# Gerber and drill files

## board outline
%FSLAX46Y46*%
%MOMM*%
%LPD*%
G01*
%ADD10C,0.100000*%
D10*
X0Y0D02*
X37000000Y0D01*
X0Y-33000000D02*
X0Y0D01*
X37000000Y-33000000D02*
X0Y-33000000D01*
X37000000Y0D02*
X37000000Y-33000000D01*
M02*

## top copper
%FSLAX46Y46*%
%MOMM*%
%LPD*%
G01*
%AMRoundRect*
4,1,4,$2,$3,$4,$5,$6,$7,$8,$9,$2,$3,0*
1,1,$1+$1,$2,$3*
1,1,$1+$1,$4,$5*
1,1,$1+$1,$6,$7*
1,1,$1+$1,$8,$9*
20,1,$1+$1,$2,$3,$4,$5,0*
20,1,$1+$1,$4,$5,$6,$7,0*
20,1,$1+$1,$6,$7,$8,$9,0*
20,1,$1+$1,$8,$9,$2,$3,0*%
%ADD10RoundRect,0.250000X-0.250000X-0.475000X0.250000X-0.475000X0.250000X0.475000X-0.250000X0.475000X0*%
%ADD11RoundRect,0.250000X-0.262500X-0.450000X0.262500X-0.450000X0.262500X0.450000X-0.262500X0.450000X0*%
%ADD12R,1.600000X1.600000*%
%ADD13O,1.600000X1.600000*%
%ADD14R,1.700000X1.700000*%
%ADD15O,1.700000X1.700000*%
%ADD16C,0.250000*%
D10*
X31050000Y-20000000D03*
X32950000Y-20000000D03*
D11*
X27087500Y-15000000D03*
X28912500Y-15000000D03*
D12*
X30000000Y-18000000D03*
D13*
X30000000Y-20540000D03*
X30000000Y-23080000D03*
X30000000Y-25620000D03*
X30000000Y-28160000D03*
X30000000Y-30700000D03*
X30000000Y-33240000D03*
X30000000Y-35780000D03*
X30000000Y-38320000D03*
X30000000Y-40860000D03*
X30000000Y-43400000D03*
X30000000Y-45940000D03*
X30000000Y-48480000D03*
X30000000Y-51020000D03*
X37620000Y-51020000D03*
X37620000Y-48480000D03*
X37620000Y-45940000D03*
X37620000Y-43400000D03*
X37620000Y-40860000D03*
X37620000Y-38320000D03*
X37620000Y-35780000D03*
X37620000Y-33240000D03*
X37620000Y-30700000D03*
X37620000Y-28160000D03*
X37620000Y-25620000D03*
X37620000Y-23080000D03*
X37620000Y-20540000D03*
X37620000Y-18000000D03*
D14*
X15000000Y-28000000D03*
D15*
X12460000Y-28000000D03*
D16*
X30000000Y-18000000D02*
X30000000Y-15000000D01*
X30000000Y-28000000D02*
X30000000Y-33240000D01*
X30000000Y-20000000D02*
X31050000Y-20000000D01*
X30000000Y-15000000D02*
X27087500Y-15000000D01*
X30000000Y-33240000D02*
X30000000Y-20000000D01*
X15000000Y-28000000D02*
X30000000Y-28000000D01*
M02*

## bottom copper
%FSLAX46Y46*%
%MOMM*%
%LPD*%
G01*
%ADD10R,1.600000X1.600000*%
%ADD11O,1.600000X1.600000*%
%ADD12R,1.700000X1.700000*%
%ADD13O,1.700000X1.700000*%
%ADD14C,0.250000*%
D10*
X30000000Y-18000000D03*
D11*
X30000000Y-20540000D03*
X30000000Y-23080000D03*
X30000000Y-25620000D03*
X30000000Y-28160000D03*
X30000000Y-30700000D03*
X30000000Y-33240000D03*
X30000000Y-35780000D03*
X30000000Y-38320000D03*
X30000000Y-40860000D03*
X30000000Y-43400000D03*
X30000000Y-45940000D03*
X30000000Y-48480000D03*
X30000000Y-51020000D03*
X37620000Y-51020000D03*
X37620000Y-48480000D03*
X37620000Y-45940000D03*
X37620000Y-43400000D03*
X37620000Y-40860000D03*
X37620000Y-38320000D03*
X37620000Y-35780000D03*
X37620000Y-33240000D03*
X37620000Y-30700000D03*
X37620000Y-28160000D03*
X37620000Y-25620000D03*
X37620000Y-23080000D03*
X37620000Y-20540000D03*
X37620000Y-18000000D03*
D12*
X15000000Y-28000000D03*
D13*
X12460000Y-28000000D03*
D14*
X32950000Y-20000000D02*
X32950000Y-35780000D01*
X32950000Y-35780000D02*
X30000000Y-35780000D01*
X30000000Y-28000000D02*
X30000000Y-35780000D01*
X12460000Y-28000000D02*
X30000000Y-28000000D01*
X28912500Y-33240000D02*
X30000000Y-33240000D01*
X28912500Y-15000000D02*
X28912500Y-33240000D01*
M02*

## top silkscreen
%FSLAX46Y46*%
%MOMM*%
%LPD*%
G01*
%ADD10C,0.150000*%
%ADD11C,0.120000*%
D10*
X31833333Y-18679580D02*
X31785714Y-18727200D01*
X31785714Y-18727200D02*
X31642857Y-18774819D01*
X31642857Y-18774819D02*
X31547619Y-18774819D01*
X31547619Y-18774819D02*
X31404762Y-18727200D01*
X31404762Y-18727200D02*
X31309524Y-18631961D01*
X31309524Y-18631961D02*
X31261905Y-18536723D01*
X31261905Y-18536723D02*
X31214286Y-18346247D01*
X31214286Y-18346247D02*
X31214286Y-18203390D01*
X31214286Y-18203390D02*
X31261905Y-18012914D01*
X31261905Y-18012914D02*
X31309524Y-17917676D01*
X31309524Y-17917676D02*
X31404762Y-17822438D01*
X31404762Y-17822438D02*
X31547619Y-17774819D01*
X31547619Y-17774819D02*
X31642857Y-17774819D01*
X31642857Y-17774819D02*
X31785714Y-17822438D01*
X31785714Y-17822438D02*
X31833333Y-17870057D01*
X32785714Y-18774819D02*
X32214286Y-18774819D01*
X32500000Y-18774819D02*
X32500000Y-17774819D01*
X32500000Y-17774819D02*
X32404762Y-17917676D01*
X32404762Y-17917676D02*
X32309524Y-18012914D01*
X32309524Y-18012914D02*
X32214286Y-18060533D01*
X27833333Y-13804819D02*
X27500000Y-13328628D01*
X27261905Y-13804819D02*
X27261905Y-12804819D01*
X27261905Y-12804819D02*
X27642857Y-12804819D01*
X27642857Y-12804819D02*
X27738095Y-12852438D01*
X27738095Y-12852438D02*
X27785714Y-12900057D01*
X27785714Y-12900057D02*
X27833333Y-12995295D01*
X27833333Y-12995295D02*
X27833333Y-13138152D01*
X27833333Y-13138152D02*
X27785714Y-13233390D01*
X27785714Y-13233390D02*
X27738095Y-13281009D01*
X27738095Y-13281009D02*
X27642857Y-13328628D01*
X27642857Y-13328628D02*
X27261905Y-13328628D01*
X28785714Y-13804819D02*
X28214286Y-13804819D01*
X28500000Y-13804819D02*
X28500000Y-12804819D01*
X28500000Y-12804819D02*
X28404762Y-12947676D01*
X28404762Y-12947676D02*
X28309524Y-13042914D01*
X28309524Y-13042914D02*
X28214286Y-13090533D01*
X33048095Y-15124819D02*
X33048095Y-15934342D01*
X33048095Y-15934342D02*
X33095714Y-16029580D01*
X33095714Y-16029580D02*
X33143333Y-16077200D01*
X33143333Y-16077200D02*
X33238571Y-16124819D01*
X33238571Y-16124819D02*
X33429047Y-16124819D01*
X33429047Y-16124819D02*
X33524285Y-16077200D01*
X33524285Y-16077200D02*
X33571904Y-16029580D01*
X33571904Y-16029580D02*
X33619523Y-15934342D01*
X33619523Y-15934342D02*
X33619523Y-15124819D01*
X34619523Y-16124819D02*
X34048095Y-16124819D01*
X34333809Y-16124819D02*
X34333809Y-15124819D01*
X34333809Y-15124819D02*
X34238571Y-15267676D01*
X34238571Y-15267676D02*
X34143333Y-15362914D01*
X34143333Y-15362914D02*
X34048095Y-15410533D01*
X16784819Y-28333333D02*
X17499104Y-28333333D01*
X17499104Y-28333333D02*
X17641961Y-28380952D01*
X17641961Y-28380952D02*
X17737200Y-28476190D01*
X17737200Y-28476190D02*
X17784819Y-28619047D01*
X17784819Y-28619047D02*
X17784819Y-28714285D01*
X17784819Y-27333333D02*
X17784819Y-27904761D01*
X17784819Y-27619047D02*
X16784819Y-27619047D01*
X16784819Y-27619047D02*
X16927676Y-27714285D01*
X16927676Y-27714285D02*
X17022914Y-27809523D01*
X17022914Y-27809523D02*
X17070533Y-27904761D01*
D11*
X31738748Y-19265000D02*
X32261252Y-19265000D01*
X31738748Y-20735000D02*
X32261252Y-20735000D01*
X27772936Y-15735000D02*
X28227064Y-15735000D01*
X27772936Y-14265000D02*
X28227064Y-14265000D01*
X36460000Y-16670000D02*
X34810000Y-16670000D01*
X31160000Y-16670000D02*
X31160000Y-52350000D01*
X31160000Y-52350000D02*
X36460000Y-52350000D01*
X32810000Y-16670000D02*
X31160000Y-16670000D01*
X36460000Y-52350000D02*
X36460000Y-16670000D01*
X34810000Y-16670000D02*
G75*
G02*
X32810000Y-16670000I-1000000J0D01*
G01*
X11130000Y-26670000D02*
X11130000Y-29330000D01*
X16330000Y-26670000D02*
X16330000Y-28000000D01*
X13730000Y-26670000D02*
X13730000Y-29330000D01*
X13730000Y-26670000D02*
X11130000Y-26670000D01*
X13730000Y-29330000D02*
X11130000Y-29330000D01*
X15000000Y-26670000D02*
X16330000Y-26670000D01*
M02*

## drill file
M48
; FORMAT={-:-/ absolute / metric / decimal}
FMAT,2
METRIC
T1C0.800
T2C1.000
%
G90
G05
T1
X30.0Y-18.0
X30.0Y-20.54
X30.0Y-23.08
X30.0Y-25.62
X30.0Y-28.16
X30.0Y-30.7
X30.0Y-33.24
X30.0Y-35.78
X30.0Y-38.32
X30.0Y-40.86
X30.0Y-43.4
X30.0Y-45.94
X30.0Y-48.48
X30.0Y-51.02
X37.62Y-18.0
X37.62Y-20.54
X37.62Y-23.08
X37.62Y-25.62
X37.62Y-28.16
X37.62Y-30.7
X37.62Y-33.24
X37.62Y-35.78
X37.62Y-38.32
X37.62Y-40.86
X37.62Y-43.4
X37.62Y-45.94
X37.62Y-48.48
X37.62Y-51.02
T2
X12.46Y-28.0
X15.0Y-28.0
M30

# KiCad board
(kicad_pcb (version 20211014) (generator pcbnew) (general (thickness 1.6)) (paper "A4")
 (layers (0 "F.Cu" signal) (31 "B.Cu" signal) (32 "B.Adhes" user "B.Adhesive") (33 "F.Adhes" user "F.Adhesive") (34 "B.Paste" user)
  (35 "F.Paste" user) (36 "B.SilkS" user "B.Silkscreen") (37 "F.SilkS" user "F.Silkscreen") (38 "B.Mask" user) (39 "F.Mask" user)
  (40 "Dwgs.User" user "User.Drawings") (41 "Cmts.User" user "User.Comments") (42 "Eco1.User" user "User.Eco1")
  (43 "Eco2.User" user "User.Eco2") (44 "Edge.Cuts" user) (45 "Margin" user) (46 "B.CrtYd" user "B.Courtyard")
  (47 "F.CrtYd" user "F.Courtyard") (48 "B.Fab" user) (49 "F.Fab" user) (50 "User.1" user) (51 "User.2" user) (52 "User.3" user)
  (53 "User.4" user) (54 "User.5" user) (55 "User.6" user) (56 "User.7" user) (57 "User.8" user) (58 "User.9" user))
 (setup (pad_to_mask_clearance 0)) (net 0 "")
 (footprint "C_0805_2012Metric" (layer "F.Cu") (at 32 20)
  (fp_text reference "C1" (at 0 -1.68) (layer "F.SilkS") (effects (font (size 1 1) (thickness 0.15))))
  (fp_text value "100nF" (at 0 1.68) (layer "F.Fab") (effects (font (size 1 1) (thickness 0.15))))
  (fp_line (start -0.261252 -0.735) (end 0.261252 -0.735) (layer "F.SilkS") (width 0.12))
  (fp_line (start -0.261252 0.735) (end 0.261252 0.735) (layer "F.SilkS") (width 0.12))
  (pad "1" smd roundrect (at -0.95 0) (size 1 1.45) (layers "F.Cu" "F.Paste" "F.Mask") (roundrect_rratio 0.25))
  (pad "2" smd roundrect (at 0.95 0) (size 1 1.45) (layers "F.Cu" "F.Paste" "F.Mask") (roundrect_rratio 0.25)))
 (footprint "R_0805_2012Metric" (layer "F.Cu") (at 28 15)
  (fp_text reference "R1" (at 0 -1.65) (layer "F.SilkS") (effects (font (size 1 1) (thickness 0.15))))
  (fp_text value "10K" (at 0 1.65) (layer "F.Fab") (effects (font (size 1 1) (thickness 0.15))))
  (fp_line (start -0.227064 0.735) (end 0.227064 0.735) (layer "F.SilkS") (width 0.12))
  (fp_line (start -0.227064 -0.735) (end 0.227064 -0.735) (layer "F.SilkS") (width 0.12))
  (pad "1" smd roundrect (at -0.9125 0) (size 1.025 1.4) (layers "F.Cu" "F.Paste" "F.Mask") (roundrect_rratio 0.243902))
  (pad "2" smd roundrect (at 0.9125 0) (size 1.025 1.4) (layers "F.Cu" "F.Paste" "F.Mask") (roundrect_rratio 0.243902)))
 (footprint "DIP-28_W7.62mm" (layer "F.Cu") (at 30 18)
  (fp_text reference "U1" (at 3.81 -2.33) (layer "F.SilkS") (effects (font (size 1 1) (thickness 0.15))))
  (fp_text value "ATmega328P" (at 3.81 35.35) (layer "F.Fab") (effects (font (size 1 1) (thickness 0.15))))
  (fp_line (start 6.46 -1.33) (end 4.81 -1.33) (layer "F.SilkS") (width 0.12))
  (fp_line (start 1.16 -1.33) (end 1.16 34.35) (layer "F.SilkS") (width 0.12))
  (fp_line (start 1.16 34.35) (end 6.46 34.35) (layer "F.SilkS") (width 0.12))
  (fp_line (start 2.81 -1.33) (end 1.16 -1.33) (layer "F.SilkS") (width 0.12))
  (fp_line (start 6.46 34.35) (end 6.46 -1.33) (layer "F.SilkS") (width 0.12))
  (fp_arc (start 4.81 -1.33) (mid 3.81 -0.33) (end 2.81 -1.33) (layer "F.SilkS") (width 0.12))
  (pad "1" thru_hole rect (at 0 0) (size 1.6 1.6) (drill 0.8) (layers *.Cu *.Mask))
  (pad "2" thru_hole oval (at 0 2.54) (size 1.6 1.6) (drill 0.8) (layers *.Cu *.Mask))
  (pad "3" thru_hole oval (at 0 5.08) (size 1.6 1.6) (drill 0.8) (layers *.Cu *.Mask))
  (pad "4" thru_hole oval (at 0 7.62) (size 1.6 1.6) (drill 0.8) (layers *.Cu *.Mask))
  (pad "5" thru_hole oval (at 0 10.16) (size 1.6 1.6) (drill 0.8) (layers *.Cu *.Mask))
  (pad "6" thru_hole oval (at 0 12.7) (size 1.6 1.6) (drill 0.8) (layers *.Cu *.Mask))
  (pad "7" thru_hole oval (at 0 15.24) (size 1.6 1.6) (drill 0.8) (layers *.Cu *.Mask))
  (pad "8" thru_hole oval (at 0 17.78) (size 1.6 1.6) (drill 0.8) (layers *.Cu *.Mask))
  (pad "9" thru_hole oval (at 0 20.32) (size 1.6 1.6) (drill 0.8) (layers *.Cu *.Mask))
  (pad "10" thru_hole oval (at 0 22.86) (size 1.6 1.6) (drill 0.8) (layers *.Cu *.Mask))
  (pad "11" thru_hole oval (at 0 25.4) (size 1.6 1.6) (drill 0.8) (layers *.Cu *.Mask))
  (pad "12" thru_hole oval (at 0 27.94) (size 1.6 1.6) (drill 0.8) (layers *.Cu *.Mask))
  (pad "13" thru_hole oval (at 0 30.48) (size 1.6 1.6) (drill 0.8) (layers *.Cu *.Mask))
  (pad "14" thru_hole oval (at 0 33.02) (size 1.6 1.6) (drill 0.8) (layers *.Cu *.Mask))
  (pad "15" thru_hole oval (at 7.62 33.02) (size 1.6 1.6) (drill 0.8) (layers *.Cu *.Mask))
  (pad "16" thru_hole oval (at 7.62 30.48) (size 1.6 1.6) (drill 0.8) (layers *.Cu *.Mask))
  (pad "17" thru_hole oval (at 7.62 27.94) (size 1.6 1.6) (drill 0.8) (layers *.Cu *.Mask))
  (pad "18" thru_hole oval (at 7.62 25.4) (size 1.6 1.6) (drill 0.8) (layers *.Cu *.Mask))
  (pad "19" thru_hole oval (at 7.62 22.86) (size 1.6 1.6) (drill 0.8) (layers *.Cu *.Mask))
  (pad "20" thru_hole oval (at 7.62 20.32) (size 1.6 1.6) (drill 0.8) (layers *.Cu *.Mask))
  (pad "21" thru_hole oval (at 7.62 17.78) (size 1.6 1.6) (drill 0.8) (layers *.Cu *.Mask))
  (pad "22" thru_hole oval (at 7.62 15.24) (size 1.6 1.6) (drill 0.8) (layers *.Cu *.Mask))
  (pad "23" thru_hole oval (at 7.62 12.7) (size 1.6 1.6) (drill 0.8) (layers *.Cu *.Mask))
  (pad "24" thru_hole oval (at 7.62 10.16) (size 1.6 1.6) (drill 0.8) (layers *.Cu *.Mask))
  (pad "25" thru_hole oval (at 7.62 7.62) (size 1.6 1.6) (drill 0.8) (layers *.Cu *.Mask))
  (pad "26" thru_hole oval (at 7.62 5.08) (size 1.6 1.6) (drill 0.8) (layers *.Cu *.Mask))
  (pad "27" thru_hole oval (at 7.62 2.54) (size 1.6 1.6) (drill 0.8) (layers *.Cu *.Mask))
  (pad "28" thru_hole oval (at 7.62 0) (size 1.6 1.6) (drill 0.8) (layers *.Cu *.Mask)))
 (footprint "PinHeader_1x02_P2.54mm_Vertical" (layer "F.Cu") (at 15 28 -90)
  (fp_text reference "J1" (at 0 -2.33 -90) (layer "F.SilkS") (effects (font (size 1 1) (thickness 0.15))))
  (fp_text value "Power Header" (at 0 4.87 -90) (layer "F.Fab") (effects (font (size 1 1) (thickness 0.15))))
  (fp_line (start -1.33 3.87) (end 1.33 3.87) (layer "F.SilkS") (width 0.12))
  (fp_line (start -1.33 -1.33) (end 0 -1.33) (layer "F.SilkS") (width 0.12))
  (fp_line (start -1.33 1.27) (end 1.33 1.27) (layer "F.SilkS") (width 0.12))
  (fp_line (start -1.33 1.27) (end -1.33 3.87) (layer "F.SilkS") (width 0.12))
  (fp_line (start 1.33 1.27) (end 1.33 3.87) (layer "F.SilkS") (width 0.12))
  (fp_line (start -1.33 0) (end -1.33 -1.33) (layer "F.SilkS") (width 0.12))
  (pad "1" thru_hole rect (at 0 0 270) (size 1.7 1.7) (drill 1) (layers *.Cu *.Mask))
  (pad "2" thru_hole oval (at 0 2.54 270) (size 1.7 1.7) (drill 1) (layers *.Cu *.Mask)))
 (gr_line (start 0 0) (end 37 0) (layer "Edge.Cuts") (width 0.1))
 (gr_line (start 0 33) (end 0 0) (layer "Edge.Cuts") (width 0.1))
 (gr_line (start 37 33) (end 0 33) (layer "Edge.Cuts") (width 0.1))
 (gr_line (start 37 0) (end 37 33) (layer "Edge.Cuts") (width 0.1))
 (segment (start 30 18) (end 30 15) (width 0.25) (layer "F.Cu") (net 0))
 (segment (start 30 28) (end 30 33.24) (width 0.25) (layer "F.Cu") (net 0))
 (segment (start 30 20) (end 31.05 20) (width 0.25) (layer "F.Cu") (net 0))
 (segment (start 30 15) (end 27.0875 15) (width 0.25) (layer "F.Cu") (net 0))
 (segment (start 30 33.24) (end 30 20) (width 0.25) (layer "F.Cu") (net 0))
 (segment (start 15 28) (end 30 28) (width 0.25) (layer "F.Cu") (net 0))
 (segment (start 32.95 20) (end 32.95 35.78) (width 0.25) (layer "B.Cu") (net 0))
 (segment (start 32.95 35.78) (end 30 35.78) (width 0.25) (layer "B.Cu") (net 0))
 (segment (start 30 28) (end 30 35.78) (width 0.25) (layer "B.Cu") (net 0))
 (segment (start 12.46 28) (end 30 28) (width 0.25) (layer "B.Cu") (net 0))
 (segment (start 28.9125 33.24) (end 30 33.24) (width 0.25) (layer "B.Cu") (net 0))
 (segment (start 28.9125 15) (end 28.9125 33.24) (width 0.25) (layer "B.Cu") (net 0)))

